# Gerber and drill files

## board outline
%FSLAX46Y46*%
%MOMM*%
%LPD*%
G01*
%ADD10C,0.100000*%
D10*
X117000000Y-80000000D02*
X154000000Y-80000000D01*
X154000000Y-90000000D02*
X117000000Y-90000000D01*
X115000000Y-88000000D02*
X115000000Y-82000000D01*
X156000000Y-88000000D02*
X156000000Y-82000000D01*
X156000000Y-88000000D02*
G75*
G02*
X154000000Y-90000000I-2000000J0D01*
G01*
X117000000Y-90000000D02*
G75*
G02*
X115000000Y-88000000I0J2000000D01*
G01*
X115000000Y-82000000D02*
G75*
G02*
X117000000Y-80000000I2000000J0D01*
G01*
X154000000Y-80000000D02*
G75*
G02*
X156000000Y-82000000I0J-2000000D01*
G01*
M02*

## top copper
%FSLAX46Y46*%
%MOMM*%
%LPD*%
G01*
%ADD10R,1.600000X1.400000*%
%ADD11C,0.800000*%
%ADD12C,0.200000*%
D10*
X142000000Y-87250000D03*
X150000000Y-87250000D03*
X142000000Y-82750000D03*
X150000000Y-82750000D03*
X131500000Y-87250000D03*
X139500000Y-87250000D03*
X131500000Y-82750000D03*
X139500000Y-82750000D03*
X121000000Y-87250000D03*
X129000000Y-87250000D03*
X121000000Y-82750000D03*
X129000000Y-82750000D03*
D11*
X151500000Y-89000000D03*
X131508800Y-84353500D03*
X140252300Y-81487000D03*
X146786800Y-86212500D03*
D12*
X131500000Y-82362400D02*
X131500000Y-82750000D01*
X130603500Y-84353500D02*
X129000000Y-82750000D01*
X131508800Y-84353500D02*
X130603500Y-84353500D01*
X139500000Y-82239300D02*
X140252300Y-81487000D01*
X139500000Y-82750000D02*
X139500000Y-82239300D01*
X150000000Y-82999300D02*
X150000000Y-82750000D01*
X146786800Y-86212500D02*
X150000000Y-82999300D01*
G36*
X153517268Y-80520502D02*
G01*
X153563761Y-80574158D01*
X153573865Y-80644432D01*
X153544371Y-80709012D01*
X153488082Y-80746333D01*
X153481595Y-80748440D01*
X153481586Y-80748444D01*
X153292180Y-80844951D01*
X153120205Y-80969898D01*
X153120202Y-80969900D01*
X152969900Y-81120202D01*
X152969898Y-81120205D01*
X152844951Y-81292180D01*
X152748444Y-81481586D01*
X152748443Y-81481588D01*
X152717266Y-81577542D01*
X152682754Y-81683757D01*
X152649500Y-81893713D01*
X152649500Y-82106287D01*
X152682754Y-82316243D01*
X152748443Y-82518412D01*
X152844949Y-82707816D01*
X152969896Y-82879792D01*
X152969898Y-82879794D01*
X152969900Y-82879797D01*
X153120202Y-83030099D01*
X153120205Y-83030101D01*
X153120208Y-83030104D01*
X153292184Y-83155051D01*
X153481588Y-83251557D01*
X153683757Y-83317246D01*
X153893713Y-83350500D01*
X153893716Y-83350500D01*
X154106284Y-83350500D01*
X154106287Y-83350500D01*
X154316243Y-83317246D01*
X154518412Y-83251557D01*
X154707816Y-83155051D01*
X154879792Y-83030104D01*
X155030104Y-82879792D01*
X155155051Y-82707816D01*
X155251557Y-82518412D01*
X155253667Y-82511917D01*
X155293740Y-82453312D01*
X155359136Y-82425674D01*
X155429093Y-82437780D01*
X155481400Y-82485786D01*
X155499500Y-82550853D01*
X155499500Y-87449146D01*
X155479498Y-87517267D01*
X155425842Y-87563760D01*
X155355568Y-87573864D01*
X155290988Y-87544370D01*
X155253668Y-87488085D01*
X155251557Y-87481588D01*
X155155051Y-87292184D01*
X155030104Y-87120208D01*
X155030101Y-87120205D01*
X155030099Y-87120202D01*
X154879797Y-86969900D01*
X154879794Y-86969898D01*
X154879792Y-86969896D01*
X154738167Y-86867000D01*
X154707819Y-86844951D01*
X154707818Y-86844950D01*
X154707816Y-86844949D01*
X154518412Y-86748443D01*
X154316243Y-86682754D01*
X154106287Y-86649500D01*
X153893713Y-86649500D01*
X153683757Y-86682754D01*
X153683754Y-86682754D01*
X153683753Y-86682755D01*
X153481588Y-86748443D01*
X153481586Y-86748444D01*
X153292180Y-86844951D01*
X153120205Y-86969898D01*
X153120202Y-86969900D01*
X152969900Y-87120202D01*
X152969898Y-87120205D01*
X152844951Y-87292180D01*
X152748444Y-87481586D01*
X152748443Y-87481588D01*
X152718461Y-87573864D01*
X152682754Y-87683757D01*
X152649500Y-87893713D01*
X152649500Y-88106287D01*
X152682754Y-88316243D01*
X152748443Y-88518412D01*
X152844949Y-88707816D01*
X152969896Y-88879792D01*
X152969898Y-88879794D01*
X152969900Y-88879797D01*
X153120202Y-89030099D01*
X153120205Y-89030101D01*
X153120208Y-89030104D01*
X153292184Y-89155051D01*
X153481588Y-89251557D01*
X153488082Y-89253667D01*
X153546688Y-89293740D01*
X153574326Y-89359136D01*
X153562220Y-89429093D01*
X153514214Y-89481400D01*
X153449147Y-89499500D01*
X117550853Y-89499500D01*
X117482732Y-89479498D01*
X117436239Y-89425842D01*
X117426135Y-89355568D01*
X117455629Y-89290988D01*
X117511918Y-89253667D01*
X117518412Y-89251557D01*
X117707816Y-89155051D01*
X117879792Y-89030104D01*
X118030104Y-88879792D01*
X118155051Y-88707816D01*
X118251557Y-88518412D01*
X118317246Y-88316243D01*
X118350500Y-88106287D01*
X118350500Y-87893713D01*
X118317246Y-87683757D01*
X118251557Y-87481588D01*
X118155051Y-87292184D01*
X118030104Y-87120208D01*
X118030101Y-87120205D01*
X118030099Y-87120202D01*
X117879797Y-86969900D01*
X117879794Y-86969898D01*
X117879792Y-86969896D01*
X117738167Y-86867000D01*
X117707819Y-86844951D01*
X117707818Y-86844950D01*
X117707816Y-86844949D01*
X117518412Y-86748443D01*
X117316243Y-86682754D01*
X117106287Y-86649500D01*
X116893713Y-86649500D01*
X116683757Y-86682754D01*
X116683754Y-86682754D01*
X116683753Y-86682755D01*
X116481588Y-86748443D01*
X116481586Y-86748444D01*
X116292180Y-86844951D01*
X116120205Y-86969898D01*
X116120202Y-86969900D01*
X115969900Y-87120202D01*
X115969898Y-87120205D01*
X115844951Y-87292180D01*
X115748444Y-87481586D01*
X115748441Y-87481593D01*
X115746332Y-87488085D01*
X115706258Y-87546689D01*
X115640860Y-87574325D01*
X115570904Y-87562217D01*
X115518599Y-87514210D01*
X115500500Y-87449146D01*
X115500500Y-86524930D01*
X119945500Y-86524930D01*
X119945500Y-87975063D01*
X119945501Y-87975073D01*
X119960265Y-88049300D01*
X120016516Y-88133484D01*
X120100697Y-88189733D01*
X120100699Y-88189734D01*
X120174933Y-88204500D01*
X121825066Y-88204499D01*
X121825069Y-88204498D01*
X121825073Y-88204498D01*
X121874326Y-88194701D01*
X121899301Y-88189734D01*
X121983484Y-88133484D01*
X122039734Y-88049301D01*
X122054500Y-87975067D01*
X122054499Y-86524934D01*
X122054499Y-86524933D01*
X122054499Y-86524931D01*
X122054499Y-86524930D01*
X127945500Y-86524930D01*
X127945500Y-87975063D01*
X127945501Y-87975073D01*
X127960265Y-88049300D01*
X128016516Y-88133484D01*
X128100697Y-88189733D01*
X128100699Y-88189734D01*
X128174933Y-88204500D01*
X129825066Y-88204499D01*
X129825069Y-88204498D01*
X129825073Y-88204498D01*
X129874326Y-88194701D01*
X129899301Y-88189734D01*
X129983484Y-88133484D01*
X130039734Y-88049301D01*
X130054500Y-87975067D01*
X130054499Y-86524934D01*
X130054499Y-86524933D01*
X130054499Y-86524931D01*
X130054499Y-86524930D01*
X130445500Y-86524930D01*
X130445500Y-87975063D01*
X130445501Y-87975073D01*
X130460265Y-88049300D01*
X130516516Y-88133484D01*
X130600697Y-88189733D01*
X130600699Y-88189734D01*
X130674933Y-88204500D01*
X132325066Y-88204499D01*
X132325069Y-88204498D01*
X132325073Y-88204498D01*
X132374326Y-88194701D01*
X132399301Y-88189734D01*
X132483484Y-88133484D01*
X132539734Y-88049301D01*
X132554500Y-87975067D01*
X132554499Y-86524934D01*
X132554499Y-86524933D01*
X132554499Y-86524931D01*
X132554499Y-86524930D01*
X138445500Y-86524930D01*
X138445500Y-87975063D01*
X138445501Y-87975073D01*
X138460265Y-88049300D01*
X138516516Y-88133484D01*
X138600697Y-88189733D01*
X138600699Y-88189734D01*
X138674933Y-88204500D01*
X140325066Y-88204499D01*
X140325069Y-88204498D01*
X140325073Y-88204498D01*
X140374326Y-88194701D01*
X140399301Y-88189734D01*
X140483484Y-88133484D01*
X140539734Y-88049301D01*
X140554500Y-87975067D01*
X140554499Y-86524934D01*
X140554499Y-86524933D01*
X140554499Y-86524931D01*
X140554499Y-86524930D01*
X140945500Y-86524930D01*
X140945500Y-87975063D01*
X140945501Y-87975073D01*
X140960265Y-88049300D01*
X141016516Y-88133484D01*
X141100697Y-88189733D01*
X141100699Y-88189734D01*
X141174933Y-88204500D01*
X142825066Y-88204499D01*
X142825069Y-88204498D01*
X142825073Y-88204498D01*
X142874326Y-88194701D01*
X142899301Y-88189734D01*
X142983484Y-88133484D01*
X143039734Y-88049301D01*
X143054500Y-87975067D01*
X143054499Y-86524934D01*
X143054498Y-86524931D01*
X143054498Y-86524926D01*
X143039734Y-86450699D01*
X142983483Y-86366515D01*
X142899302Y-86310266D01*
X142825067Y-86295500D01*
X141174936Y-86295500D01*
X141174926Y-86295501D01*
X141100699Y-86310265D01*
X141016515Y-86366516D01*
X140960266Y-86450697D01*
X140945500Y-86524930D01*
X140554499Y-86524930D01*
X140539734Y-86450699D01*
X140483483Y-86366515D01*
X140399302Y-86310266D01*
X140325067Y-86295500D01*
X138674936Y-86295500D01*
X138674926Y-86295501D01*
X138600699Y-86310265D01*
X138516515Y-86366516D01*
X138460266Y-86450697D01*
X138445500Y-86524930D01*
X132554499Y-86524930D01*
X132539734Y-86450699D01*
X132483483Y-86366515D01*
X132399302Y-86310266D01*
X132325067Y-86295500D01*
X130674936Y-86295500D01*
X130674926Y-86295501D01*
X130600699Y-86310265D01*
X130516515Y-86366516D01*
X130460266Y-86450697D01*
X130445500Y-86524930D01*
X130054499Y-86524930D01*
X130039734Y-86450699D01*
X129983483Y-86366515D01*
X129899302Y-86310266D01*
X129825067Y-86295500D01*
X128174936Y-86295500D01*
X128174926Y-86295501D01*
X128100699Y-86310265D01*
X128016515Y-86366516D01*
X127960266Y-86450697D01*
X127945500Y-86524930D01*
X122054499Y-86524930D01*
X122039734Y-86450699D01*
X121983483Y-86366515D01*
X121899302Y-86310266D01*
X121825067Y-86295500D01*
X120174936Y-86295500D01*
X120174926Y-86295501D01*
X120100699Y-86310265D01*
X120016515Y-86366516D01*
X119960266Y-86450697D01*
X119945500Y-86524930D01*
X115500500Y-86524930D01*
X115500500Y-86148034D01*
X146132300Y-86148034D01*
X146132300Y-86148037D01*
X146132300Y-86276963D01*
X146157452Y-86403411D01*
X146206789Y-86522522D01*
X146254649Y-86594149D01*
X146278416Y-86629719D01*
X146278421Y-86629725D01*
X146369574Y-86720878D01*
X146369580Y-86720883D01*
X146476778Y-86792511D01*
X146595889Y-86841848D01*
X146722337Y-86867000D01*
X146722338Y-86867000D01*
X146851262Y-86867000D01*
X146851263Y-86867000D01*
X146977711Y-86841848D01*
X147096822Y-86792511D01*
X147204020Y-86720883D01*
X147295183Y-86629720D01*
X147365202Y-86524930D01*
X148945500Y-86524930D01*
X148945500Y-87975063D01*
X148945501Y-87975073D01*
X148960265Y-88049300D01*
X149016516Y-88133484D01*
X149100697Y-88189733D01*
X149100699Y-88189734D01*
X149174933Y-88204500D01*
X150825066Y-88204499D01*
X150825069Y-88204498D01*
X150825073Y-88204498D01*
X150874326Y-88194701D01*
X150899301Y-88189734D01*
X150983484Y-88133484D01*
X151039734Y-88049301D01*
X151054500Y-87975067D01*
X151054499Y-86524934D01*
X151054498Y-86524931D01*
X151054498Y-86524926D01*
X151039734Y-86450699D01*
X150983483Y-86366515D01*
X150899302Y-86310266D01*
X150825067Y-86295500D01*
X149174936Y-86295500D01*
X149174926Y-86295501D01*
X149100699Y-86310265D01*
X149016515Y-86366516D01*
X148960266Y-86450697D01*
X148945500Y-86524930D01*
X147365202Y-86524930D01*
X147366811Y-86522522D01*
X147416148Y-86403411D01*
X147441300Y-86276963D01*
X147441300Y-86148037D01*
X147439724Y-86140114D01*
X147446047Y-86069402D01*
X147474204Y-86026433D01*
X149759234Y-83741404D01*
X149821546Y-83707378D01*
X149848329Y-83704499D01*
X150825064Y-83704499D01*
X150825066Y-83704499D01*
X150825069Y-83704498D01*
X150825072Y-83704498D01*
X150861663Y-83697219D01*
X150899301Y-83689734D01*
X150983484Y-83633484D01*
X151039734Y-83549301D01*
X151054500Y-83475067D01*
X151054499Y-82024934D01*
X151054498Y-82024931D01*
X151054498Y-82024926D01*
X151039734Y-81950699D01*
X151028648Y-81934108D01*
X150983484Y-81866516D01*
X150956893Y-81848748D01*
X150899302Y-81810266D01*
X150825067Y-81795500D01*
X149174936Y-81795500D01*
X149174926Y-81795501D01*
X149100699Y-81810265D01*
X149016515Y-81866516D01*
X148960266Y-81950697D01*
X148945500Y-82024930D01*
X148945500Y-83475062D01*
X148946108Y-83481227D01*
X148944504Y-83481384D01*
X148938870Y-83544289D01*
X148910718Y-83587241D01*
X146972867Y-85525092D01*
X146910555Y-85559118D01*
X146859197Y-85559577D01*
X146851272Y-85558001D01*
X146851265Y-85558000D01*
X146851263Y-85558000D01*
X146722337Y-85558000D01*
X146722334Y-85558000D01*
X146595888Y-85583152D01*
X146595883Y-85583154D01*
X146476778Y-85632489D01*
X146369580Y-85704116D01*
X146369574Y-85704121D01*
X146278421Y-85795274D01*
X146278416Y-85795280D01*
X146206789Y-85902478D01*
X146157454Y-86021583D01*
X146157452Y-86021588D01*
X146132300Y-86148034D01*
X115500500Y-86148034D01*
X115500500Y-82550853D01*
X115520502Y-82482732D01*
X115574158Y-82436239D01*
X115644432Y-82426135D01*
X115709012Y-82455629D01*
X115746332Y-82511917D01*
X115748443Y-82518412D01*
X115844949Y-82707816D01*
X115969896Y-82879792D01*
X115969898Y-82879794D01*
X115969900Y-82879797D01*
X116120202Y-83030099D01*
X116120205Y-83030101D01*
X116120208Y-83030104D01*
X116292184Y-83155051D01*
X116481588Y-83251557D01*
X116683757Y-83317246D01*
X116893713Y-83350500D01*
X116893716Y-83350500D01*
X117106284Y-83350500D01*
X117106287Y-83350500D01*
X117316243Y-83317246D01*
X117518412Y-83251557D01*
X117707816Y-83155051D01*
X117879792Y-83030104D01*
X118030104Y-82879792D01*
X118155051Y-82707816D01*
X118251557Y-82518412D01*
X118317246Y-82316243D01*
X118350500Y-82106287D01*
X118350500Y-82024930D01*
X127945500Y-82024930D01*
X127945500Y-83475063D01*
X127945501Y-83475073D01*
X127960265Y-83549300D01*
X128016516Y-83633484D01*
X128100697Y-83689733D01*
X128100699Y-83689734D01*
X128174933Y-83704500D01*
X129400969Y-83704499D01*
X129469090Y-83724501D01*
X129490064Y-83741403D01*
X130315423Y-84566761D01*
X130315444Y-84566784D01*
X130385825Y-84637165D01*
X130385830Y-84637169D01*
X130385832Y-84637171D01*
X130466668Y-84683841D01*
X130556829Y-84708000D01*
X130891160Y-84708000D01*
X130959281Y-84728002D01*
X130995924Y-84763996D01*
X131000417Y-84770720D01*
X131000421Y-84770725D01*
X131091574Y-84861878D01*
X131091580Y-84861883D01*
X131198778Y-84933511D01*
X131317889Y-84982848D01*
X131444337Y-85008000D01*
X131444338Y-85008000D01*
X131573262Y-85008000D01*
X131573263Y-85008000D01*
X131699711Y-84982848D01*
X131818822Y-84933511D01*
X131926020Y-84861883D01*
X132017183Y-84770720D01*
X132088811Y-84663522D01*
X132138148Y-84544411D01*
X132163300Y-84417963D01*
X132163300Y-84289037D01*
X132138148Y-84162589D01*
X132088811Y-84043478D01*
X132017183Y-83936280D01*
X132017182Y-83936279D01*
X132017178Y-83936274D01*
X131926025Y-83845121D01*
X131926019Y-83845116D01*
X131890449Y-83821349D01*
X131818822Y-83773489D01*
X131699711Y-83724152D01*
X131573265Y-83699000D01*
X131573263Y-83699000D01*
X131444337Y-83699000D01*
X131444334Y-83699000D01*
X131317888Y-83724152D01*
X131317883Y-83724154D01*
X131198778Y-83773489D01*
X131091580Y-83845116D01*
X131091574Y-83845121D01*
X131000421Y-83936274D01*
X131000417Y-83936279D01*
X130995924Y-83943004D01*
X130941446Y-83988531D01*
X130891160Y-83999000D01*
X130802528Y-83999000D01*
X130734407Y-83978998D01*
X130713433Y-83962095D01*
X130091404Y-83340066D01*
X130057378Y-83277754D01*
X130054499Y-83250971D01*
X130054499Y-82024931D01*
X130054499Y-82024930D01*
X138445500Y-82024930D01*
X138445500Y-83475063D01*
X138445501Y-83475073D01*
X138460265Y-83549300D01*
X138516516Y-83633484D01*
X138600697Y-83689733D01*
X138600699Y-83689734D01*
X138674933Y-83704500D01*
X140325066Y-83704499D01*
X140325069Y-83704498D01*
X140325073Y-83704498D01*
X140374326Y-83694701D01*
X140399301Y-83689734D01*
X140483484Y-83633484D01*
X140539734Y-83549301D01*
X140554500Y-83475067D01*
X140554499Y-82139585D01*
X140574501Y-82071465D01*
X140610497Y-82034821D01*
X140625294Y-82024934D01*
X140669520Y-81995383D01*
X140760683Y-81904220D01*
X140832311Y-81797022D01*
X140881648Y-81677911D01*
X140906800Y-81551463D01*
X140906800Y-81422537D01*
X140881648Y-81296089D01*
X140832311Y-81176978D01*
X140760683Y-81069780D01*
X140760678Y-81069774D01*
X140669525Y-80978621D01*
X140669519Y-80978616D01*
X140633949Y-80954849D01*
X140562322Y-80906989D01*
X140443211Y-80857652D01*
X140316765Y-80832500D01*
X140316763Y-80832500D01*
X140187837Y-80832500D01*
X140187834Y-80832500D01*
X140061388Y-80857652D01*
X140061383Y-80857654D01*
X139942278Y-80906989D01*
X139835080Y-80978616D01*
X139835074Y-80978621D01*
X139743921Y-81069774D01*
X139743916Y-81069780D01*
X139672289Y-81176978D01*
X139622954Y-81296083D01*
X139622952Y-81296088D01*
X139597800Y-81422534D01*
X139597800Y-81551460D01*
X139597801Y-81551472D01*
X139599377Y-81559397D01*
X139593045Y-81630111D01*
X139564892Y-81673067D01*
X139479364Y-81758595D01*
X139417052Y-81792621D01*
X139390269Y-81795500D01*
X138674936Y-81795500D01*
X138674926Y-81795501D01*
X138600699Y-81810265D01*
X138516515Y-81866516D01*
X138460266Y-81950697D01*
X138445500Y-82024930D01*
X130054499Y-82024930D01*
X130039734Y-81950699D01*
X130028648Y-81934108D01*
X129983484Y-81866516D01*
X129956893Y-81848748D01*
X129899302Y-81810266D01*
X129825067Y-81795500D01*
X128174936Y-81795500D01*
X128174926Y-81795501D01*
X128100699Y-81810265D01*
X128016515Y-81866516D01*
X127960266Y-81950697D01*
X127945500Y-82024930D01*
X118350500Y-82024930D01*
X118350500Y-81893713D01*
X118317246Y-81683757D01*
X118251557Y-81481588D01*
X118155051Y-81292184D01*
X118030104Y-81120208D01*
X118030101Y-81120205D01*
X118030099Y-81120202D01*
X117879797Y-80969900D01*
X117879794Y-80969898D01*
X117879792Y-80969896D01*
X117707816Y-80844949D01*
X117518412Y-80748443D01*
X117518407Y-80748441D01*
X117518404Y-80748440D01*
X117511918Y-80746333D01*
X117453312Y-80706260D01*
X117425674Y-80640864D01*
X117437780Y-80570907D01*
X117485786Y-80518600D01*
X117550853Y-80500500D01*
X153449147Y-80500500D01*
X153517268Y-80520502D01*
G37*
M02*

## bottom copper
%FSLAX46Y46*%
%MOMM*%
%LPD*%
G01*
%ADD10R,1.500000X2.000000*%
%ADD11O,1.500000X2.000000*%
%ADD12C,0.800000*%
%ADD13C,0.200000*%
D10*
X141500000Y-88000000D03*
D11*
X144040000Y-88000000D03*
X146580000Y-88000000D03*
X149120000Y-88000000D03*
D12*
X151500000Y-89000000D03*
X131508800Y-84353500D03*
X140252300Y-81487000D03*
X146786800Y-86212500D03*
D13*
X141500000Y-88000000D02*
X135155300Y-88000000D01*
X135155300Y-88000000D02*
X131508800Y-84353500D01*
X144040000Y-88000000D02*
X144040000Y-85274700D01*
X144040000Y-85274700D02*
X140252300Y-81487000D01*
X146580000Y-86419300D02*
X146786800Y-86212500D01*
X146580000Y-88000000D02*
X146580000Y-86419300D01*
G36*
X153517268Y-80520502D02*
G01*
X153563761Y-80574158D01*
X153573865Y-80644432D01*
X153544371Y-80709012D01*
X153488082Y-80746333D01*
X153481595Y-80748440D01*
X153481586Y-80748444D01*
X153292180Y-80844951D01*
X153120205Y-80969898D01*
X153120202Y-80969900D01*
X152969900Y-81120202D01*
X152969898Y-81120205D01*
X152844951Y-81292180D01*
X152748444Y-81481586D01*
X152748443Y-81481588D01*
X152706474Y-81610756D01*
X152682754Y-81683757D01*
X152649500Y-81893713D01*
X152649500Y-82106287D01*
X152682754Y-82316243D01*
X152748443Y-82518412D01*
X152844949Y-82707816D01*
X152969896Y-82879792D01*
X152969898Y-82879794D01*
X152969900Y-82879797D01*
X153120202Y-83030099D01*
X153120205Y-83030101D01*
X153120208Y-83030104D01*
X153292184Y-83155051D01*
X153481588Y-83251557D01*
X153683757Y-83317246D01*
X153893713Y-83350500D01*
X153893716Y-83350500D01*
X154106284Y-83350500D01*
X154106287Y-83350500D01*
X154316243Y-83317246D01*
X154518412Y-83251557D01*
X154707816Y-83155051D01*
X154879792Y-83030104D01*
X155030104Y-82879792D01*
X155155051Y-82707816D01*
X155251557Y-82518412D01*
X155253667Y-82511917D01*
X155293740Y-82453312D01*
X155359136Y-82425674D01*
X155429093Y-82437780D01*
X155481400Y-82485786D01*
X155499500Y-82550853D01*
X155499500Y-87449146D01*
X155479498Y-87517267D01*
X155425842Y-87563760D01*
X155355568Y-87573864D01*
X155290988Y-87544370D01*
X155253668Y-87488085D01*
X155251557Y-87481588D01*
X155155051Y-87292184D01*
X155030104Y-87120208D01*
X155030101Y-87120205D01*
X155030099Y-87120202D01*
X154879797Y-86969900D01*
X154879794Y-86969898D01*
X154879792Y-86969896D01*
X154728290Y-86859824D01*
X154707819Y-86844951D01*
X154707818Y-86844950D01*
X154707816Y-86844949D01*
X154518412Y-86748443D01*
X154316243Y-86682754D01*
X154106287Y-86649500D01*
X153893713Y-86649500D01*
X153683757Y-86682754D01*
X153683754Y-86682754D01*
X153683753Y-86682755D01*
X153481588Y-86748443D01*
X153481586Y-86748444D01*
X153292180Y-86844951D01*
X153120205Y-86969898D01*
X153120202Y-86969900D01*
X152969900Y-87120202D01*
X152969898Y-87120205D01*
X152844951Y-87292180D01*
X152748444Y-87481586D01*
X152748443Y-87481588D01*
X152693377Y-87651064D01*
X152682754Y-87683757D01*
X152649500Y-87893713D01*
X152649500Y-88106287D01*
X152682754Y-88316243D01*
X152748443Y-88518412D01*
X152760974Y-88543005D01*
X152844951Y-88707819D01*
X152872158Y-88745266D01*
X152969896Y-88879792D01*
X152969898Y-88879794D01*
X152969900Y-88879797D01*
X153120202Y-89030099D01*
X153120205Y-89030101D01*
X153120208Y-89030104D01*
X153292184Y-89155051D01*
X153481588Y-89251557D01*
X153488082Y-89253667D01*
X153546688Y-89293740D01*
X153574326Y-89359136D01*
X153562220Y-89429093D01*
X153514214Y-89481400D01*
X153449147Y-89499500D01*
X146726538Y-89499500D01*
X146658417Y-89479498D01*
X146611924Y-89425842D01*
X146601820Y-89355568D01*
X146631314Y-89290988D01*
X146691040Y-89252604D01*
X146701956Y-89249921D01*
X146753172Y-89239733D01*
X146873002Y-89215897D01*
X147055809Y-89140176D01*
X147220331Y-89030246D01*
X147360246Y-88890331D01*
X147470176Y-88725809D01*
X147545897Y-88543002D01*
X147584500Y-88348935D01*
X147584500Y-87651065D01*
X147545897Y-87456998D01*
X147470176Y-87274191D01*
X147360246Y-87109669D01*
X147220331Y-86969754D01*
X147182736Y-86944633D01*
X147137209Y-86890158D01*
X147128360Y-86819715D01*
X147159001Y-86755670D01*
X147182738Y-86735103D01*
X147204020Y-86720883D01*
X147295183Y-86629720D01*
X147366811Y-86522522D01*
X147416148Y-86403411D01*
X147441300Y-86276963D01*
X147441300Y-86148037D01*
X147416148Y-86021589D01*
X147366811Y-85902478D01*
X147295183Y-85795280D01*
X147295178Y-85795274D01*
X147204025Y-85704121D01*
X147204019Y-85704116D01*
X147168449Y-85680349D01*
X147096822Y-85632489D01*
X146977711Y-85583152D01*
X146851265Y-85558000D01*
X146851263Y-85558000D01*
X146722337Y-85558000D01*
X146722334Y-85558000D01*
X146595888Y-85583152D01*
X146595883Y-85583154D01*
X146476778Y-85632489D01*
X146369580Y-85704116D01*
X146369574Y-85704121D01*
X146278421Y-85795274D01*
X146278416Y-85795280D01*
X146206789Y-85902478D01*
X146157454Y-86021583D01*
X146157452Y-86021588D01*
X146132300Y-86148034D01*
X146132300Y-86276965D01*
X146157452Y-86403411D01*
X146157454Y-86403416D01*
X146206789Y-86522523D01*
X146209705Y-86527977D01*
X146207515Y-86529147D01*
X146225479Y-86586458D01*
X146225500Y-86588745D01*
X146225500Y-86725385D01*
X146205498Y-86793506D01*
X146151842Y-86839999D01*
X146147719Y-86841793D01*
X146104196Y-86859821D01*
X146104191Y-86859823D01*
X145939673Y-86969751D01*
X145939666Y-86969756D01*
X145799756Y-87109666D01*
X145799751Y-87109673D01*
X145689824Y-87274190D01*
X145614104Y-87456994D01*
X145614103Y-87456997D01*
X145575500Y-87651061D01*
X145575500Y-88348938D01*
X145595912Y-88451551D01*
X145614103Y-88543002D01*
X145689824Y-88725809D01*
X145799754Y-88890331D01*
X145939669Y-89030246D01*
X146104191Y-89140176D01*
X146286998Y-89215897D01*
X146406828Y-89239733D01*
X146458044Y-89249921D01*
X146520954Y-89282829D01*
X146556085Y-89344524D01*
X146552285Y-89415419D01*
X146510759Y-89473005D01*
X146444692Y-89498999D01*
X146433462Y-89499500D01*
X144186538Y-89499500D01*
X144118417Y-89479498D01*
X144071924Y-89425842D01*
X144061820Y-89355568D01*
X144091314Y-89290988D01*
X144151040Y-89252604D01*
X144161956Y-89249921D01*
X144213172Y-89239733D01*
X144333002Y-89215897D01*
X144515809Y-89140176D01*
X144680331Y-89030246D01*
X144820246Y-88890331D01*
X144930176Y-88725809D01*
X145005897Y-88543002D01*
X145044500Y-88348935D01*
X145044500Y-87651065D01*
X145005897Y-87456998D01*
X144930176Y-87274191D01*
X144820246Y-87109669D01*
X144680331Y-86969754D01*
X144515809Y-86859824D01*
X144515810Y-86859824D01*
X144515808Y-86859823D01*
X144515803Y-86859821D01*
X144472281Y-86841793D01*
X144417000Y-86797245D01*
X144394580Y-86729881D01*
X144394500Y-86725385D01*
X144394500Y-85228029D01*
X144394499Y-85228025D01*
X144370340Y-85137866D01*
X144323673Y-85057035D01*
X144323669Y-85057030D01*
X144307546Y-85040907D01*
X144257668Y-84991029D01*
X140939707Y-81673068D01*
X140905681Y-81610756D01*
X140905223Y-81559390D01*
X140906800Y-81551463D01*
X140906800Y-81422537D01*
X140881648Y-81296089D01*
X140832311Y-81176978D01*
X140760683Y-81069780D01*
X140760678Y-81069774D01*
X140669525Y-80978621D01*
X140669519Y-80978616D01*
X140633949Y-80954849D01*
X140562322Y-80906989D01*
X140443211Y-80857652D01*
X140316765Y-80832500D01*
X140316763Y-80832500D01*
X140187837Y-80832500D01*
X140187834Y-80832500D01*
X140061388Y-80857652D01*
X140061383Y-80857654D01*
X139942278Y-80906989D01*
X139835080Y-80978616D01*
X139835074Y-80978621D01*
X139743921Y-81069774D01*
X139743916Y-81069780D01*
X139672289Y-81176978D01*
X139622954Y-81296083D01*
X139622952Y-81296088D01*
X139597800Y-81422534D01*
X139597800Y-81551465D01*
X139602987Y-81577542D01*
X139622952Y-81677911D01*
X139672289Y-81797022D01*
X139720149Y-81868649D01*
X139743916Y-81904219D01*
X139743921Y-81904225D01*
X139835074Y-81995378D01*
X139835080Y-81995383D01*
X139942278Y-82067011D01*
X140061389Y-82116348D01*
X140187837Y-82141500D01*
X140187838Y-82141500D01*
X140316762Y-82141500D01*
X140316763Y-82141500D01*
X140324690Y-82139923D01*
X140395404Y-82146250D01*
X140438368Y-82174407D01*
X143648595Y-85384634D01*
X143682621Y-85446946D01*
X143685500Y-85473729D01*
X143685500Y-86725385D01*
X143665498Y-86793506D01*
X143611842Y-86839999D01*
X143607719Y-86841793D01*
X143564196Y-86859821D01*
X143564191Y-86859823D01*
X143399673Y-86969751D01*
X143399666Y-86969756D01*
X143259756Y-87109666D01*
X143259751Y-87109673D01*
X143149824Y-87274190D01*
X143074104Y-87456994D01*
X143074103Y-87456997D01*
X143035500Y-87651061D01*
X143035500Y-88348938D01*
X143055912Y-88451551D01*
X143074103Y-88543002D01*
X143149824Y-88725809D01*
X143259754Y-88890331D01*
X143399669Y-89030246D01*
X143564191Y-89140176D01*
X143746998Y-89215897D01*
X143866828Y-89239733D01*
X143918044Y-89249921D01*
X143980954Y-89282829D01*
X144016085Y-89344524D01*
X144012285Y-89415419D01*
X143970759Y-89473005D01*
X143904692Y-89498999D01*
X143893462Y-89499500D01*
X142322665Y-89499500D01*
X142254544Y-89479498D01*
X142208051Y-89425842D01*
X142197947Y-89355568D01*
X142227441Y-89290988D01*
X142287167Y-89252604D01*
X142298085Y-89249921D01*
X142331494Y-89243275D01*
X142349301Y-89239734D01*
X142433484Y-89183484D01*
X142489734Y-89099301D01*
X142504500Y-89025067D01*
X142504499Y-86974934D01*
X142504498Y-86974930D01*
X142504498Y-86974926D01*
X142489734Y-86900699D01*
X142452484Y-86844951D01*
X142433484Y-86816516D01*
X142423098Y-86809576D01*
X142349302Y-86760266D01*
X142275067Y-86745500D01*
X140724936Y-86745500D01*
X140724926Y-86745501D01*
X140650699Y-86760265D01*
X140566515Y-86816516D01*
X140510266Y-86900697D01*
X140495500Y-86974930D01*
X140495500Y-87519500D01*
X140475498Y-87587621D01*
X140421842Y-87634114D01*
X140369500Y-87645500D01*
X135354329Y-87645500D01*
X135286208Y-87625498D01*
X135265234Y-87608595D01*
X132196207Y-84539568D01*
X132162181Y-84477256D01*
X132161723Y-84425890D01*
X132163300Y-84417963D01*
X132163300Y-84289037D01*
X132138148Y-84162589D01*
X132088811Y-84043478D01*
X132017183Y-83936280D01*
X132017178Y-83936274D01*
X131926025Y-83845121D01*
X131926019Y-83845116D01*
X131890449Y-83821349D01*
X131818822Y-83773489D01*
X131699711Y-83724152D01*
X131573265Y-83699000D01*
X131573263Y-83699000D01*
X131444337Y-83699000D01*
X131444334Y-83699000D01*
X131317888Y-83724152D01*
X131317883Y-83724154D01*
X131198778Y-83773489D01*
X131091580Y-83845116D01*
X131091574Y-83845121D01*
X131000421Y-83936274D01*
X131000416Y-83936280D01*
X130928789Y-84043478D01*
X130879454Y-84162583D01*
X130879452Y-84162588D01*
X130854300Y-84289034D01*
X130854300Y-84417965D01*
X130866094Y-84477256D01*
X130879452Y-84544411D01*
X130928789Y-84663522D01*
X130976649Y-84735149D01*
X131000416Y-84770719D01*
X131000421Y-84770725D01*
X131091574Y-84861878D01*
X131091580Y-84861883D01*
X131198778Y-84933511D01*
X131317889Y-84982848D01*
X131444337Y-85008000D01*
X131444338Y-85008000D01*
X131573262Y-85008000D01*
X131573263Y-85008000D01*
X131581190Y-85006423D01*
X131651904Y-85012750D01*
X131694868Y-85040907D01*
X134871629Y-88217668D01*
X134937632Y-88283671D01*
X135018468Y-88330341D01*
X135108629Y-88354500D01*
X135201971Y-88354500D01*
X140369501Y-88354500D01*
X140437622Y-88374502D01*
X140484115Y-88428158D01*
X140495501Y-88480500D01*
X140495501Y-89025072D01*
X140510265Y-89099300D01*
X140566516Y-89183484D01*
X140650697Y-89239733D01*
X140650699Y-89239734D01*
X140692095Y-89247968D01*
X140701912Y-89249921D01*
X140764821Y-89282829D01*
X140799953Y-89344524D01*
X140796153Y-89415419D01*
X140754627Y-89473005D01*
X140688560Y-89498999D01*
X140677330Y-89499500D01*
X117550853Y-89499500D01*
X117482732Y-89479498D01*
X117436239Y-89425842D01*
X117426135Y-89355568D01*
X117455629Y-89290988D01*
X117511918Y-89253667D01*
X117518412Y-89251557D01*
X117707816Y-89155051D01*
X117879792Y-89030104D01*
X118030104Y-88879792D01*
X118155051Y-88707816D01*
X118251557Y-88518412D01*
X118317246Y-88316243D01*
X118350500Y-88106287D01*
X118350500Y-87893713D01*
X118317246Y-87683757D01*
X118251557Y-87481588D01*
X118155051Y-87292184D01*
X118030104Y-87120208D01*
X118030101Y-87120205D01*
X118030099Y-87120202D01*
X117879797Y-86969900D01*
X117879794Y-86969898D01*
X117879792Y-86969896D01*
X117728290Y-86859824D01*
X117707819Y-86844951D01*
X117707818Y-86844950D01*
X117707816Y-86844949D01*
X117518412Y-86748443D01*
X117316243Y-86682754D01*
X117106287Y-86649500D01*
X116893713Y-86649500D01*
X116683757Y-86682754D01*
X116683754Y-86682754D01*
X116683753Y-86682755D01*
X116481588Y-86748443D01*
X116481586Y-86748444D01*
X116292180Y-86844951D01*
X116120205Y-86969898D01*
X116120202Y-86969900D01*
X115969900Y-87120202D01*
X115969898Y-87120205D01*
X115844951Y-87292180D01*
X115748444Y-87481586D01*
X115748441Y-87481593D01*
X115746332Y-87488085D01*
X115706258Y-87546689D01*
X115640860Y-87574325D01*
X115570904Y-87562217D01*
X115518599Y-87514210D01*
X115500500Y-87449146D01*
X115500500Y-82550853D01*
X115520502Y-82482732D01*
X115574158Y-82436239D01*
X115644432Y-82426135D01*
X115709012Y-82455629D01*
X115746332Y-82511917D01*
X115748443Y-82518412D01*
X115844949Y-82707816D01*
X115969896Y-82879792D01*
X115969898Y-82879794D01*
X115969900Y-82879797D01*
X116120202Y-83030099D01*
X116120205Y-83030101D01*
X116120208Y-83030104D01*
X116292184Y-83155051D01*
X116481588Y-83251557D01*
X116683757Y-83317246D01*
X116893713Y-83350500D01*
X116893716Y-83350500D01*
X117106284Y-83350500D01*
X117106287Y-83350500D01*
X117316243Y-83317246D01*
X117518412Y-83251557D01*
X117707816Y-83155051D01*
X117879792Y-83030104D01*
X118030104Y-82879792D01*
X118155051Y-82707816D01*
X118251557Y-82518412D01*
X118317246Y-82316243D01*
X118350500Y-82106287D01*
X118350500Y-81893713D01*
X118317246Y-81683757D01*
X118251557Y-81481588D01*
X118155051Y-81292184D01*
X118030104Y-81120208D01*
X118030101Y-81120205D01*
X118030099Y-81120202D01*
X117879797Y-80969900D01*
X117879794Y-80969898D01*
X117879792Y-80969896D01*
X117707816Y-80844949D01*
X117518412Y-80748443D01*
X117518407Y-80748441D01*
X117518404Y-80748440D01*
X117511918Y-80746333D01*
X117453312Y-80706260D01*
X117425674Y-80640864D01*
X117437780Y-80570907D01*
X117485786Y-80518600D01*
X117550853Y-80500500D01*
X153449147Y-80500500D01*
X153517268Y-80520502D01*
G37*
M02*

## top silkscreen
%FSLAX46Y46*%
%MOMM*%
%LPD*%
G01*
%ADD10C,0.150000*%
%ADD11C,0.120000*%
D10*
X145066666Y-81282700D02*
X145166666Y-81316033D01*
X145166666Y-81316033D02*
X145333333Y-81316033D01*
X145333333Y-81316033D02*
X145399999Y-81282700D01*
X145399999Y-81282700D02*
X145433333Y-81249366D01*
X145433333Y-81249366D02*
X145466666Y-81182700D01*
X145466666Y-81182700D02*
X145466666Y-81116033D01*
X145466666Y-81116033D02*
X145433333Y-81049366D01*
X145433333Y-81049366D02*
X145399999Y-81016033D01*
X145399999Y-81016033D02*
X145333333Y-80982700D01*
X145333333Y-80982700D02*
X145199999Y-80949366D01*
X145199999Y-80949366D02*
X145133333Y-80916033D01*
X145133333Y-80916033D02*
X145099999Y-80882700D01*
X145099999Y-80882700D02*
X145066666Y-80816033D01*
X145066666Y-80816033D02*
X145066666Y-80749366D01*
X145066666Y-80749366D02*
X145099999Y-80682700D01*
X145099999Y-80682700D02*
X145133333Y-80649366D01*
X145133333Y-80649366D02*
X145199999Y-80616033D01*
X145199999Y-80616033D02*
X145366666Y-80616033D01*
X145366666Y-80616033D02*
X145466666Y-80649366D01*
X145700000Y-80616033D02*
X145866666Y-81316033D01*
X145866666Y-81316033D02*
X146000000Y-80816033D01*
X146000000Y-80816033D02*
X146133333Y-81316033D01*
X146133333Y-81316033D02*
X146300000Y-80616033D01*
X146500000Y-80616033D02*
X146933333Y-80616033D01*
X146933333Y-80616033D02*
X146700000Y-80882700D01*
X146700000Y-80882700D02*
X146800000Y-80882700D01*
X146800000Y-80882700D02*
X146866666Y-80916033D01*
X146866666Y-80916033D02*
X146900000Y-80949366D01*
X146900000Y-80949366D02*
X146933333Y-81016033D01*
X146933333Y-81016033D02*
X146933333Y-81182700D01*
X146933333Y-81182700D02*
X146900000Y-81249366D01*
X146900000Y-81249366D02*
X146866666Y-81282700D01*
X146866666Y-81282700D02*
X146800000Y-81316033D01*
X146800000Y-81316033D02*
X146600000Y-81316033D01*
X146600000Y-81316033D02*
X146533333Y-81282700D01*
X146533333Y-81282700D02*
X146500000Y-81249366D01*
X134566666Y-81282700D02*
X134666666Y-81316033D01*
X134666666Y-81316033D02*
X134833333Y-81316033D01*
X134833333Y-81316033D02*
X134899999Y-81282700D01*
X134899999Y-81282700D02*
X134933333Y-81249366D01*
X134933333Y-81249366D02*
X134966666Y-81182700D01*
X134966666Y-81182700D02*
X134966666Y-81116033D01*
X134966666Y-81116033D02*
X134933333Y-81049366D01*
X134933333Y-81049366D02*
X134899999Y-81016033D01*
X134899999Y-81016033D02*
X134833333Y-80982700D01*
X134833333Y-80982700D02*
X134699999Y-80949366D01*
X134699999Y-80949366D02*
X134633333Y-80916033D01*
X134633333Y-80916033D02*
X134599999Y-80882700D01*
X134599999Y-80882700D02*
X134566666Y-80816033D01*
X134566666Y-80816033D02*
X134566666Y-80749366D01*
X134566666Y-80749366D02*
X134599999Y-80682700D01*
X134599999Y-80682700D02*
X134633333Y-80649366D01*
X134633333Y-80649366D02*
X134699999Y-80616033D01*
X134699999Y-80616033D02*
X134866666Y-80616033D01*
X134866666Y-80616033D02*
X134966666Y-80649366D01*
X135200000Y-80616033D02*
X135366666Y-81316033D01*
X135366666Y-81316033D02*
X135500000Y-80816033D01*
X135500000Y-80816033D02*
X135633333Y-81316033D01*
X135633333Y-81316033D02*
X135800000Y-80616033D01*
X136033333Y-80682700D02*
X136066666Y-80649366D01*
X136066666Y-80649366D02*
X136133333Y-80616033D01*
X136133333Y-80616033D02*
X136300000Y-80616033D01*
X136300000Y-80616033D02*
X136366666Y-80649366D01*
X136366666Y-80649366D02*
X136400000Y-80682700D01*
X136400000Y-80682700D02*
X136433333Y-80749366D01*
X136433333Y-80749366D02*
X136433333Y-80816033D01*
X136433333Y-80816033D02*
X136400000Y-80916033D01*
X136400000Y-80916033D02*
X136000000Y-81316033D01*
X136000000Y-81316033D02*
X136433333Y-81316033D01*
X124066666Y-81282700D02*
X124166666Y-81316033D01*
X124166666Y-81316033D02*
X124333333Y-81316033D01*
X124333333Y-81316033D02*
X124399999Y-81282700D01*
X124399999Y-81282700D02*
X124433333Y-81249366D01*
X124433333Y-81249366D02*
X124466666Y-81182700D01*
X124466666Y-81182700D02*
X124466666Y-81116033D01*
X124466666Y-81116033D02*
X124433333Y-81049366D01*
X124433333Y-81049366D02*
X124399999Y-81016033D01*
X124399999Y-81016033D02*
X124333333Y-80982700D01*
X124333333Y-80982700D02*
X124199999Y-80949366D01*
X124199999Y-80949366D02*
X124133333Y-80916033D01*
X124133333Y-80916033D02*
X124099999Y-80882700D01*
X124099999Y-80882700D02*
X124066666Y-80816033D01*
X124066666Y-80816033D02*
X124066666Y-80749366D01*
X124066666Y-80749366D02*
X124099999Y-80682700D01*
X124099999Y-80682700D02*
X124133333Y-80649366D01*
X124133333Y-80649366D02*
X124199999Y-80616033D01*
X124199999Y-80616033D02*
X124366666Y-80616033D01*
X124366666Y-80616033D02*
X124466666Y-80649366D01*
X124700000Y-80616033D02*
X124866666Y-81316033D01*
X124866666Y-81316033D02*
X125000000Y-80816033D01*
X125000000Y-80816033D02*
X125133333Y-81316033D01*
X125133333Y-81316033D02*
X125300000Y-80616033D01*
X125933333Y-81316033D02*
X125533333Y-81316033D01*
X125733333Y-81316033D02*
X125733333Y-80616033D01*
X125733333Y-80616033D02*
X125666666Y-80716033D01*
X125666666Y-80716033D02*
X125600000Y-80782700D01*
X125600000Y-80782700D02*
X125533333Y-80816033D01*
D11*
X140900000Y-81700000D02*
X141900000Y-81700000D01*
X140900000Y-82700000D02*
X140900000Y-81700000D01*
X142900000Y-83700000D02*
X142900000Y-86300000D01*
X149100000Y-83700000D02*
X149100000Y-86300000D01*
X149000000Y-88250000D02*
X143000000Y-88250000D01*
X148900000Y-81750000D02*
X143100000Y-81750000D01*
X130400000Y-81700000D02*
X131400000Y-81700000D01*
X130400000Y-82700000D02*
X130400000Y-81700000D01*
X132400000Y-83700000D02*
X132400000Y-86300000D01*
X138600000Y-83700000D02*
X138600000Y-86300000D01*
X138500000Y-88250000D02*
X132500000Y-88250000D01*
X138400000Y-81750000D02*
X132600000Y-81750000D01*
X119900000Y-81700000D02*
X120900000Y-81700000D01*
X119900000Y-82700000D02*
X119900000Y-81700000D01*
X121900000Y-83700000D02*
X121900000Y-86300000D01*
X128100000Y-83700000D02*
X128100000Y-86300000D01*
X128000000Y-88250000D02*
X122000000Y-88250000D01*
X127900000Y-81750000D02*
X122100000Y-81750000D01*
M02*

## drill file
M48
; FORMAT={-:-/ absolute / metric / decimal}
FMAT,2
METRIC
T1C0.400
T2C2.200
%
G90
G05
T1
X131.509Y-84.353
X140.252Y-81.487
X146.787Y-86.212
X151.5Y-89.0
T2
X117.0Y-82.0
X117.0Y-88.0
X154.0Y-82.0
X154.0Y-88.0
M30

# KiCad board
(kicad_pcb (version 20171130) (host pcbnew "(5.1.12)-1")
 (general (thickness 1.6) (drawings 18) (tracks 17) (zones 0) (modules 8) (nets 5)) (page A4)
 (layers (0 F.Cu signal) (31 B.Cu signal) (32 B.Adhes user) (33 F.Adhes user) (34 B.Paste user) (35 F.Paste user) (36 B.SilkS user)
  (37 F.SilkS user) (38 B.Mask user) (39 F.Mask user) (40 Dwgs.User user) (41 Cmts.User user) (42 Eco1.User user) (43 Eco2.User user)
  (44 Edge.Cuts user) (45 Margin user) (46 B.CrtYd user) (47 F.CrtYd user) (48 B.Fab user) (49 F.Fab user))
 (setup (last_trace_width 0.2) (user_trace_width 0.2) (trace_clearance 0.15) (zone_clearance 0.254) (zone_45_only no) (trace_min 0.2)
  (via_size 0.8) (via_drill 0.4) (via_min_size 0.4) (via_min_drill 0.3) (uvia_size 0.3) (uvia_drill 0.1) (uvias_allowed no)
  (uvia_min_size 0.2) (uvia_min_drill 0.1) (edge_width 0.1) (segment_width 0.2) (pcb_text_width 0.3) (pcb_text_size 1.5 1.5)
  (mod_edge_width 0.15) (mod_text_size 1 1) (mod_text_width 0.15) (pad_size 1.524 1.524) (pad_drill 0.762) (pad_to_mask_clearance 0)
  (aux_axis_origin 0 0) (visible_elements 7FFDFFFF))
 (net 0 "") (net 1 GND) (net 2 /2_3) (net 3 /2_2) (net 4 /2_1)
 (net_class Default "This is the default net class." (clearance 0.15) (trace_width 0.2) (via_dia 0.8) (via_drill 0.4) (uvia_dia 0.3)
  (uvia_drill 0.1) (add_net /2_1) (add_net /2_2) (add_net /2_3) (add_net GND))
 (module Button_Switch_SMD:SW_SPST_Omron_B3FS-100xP (layer F.Cu) (at 146 85)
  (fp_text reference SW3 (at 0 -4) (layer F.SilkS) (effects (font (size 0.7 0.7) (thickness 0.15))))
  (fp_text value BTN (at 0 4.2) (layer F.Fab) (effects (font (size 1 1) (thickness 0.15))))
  (fp_line (start -5.1 -3.3) (end -4.1 -3.3) (layer F.SilkS) (width 0.12))
  (fp_line (start -5.1 -2.3) (end -5.1 -3.3) (layer F.SilkS) (width 0.12))
  (fp_line (start -3.1 -1.3) (end -3.1 1.3) (layer F.SilkS) (width 0.12))
  (fp_line (start 3.1 -1.3) (end 3.1 1.3) (layer F.SilkS) (width 0.12))
  (fp_line (start 3 3.25) (end -3 3.25) (layer F.SilkS) (width 0.12))
  (fp_line (start 2.9 -3.25) (end -2.9 -3.25) (layer F.SilkS) (width 0.12))
  (pad 3 smd rect (at -4 2.25 180) (size 1.6 1.4) (layers F.Cu F.Paste F.Mask))
  (pad 4 smd rect (at 4 2.25 180) (size 1.6 1.4) (layers F.Cu F.Paste F.Mask))
  (pad 1 smd rect (at -4 -2.25 180) (size 1.6 1.4) (layers F.Cu F.Paste F.Mask) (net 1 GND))
  (pad 2 smd rect (at 4 -2.25 180) (size 1.6 1.4) (layers F.Cu F.Paste F.Mask) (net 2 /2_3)))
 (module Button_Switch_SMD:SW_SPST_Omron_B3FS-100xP (layer F.Cu) (at 135.5 85)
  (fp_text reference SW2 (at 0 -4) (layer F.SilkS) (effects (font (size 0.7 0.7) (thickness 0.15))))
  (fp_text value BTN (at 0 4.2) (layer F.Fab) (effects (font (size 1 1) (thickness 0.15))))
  (fp_line (start -5.1 -3.3) (end -4.1 -3.3) (layer F.SilkS) (width 0.12))
  (fp_line (start -5.1 -2.3) (end -5.1 -3.3) (layer F.SilkS) (width 0.12))
  (fp_line (start -3.1 -1.3) (end -3.1 1.3) (layer F.SilkS) (width 0.12))
  (fp_line (start 3.1 -1.3) (end 3.1 1.3) (layer F.SilkS) (width 0.12))
  (fp_line (start 3 3.25) (end -3 3.25) (layer F.SilkS) (width 0.12))
  (fp_line (start 2.9 -3.25) (end -2.9 -3.25) (layer F.SilkS) (width 0.12))
  (pad 3 smd rect (at -4 2.25 180) (size 1.6 1.4) (layers F.Cu F.Paste F.Mask))
  (pad 4 smd rect (at 4 2.25 180) (size 1.6 1.4) (layers F.Cu F.Paste F.Mask))
  (pad 1 smd rect (at -4 -2.25 180) (size 1.6 1.4) (layers F.Cu F.Paste F.Mask) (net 1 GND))
  (pad 2 smd rect (at 4 -2.25 180) (size 1.6 1.4) (layers F.Cu F.Paste F.Mask) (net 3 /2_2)))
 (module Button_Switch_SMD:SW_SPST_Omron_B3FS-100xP (layer F.Cu) (at 125 85)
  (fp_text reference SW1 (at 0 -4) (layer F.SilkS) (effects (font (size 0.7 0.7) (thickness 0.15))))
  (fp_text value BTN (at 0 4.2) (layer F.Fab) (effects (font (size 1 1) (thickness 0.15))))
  (fp_line (start -5.1 -3.3) (end -4.1 -3.3) (layer F.SilkS) (width 0.12))
  (fp_line (start -5.1 -2.3) (end -5.1 -3.3) (layer F.SilkS) (width 0.12))
  (fp_line (start -3.1 -1.3) (end -3.1 1.3) (layer F.SilkS) (width 0.12))
  (fp_line (start 3.1 -1.3) (end 3.1 1.3) (layer F.SilkS) (width 0.12))
  (fp_line (start 3 3.25) (end -3 3.25) (layer F.SilkS) (width 0.12))
  (fp_line (start 2.9 -3.25) (end -2.9 -3.25) (layer F.SilkS) (width 0.12))
  (pad 3 smd rect (at -4 2.25 180) (size 1.6 1.4) (layers F.Cu F.Paste F.Mask))
  (pad 4 smd rect (at 4 2.25 180) (size 1.6 1.4) (layers F.Cu F.Paste F.Mask))
  (pad 1 smd rect (at -4 -2.25 180) (size 1.6 1.4) (layers F.Cu F.Paste F.Mask) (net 1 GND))
  (pad 2 smd rect (at 4 -2.25 180) (size 1.6 1.4) (layers F.Cu F.Paste F.Mask) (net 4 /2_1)))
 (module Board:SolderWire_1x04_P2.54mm (layer B.Cu) (at 141.5 88 270)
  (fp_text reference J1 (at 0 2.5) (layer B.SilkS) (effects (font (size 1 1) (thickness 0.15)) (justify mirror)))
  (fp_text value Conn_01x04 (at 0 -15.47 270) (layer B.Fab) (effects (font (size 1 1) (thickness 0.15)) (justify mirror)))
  (pad 1 smd rect (at 0 0 270) (size 2 1.5) (layers B.Cu B.Paste B.Mask) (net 4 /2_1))
  (pad 2 smd oval (at 0 -2.54 270) (size 2 1.5) (layers B.Cu B.Paste B.Mask) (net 3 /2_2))
  (pad 3 smd oval (at 0 -5.08 270) (size 2 1.5) (layers B.Cu B.Paste B.Mask) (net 2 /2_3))
  (pad 4 smd oval (at 0 -7.62 270) (size 2 1.5) (layers B.Cu B.Paste B.Mask) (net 1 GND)))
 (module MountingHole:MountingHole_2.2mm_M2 (layer F.Cu) (at 117 88)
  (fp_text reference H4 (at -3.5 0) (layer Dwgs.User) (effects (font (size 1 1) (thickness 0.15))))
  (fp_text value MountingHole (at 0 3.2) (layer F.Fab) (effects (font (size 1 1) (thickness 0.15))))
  (pad 1 np_thru_hole circle (at 0 0) (size 2.2 2.2) (drill 2.2) (layers *.Cu *.Mask)))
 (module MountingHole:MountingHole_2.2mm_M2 (layer F.Cu) (at 154 88)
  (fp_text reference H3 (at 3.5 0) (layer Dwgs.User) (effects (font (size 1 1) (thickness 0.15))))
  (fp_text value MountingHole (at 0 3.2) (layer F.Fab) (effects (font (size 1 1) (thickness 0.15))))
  (pad 1 np_thru_hole circle (at 0 0) (size 2.2 2.2) (drill 2.2) (layers *.Cu *.Mask)))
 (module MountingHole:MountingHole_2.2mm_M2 (layer F.Cu) (at 154 82)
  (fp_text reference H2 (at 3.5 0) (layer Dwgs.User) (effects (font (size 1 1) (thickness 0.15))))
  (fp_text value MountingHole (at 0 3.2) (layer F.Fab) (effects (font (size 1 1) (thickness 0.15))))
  (pad 1 np_thru_hole circle (at 0 0) (size 2.2 2.2) (drill 2.2) (layers *.Cu *.Mask)))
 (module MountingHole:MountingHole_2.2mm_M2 (layer F.Cu) (at 117 82)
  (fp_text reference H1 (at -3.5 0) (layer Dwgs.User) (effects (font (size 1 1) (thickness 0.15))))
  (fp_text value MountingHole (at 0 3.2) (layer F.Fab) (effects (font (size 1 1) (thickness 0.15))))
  (pad 1 np_thru_hole circle (at 0 0) (size 2.2 2.2) (drill 2.2) (layers *.Cu *.Mask)))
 (gr_line (start 117 80) (end 154 80) (layer Edge.Cuts) (width 0.1))
 (gr_line (start 154 90) (end 117 90) (layer Edge.Cuts) (width 0.1))
 (gr_line (start 115 88) (end 115 82) (layer Edge.Cuts) (width 0.1))
 (gr_line (start 156 88) (end 156 82) (layer Edge.Cuts) (width 0.1))
 (gr_arc (start 154 88) (end 154 90) (angle -90) (layer Edge.Cuts) (width 0.1))
 (gr_arc (start 117 88) (end 115 88) (angle -90) (layer Edge.Cuts) (width 0.1))
 (gr_arc (start 117 82) (end 117 80) (angle -90) (layer Edge.Cuts) (width 0.1))
 (gr_arc (start 154 82) (end 156 82) (angle -90) (layer Edge.Cuts) (width 0.1))
 (segment (start 131.5 82.3624) (end 131.5 82.75) (width 0.2) (layer F.Cu) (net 1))
 (via (at 151.5 89) (size 0.8) (layers F.Cu B.Cu) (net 1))
 (segment (start 141.5 88) (end 135.1553 88) (width 0.2) (layer B.Cu) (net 4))
 (segment (start 135.1553 88) (end 131.5088 84.3535) (width 0.2) (layer B.Cu) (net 4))
 (via (at 131.5088 84.3535) (size 0.8) (layers F.Cu B.Cu) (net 4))
 (segment (start 130.6035 84.3535) (end 129 82.75) (width 0.2) (layer F.Cu) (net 4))
 (segment (start 131.5088 84.3535) (end 130.6035 84.3535) (width 0.2) (layer F.Cu) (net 4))
 (segment (start 144.04 88) (end 144.04 85.2747) (width 0.2) (layer B.Cu) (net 3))
 (segment (start 144.04 85.2747) (end 140.2523 81.487) (width 0.2) (layer B.Cu) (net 3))
 (via (at 140.2523 81.487) (size 0.8) (layers F.Cu B.Cu) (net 3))
 (segment (start 139.5 82.2393) (end 140.2523 81.487) (width 0.2) (layer F.Cu) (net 3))
 (segment (start 139.5 82.75) (end 139.5 82.2393) (width 0.2) (layer F.Cu) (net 3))
 (via (at 146.7868 86.2125) (size 0.8) (layers F.Cu B.Cu) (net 2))
 (segment (start 150 82.9993) (end 150 82.75) (width 0.2) (layer F.Cu) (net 2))
 (segment (start 146.7868 86.2125) (end 150 82.9993) (width 0.2) (layer F.Cu) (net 2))
 (segment (start 146.58 86.4193) (end 146.7868 86.2125) (width 0.2) (layer B.Cu) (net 2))
 (segment (start 146.58 88) (end 146.58 86.4193) (width 0.2) (layer B.Cu) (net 2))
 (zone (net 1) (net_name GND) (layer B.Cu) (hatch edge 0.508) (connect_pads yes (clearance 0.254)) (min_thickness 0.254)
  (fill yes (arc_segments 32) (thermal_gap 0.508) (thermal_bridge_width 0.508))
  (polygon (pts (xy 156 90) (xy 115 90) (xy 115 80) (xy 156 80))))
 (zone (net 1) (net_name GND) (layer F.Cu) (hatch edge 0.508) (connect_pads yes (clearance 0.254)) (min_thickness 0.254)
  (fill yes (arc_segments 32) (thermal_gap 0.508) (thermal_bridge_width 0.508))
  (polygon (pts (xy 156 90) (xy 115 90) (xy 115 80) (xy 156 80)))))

